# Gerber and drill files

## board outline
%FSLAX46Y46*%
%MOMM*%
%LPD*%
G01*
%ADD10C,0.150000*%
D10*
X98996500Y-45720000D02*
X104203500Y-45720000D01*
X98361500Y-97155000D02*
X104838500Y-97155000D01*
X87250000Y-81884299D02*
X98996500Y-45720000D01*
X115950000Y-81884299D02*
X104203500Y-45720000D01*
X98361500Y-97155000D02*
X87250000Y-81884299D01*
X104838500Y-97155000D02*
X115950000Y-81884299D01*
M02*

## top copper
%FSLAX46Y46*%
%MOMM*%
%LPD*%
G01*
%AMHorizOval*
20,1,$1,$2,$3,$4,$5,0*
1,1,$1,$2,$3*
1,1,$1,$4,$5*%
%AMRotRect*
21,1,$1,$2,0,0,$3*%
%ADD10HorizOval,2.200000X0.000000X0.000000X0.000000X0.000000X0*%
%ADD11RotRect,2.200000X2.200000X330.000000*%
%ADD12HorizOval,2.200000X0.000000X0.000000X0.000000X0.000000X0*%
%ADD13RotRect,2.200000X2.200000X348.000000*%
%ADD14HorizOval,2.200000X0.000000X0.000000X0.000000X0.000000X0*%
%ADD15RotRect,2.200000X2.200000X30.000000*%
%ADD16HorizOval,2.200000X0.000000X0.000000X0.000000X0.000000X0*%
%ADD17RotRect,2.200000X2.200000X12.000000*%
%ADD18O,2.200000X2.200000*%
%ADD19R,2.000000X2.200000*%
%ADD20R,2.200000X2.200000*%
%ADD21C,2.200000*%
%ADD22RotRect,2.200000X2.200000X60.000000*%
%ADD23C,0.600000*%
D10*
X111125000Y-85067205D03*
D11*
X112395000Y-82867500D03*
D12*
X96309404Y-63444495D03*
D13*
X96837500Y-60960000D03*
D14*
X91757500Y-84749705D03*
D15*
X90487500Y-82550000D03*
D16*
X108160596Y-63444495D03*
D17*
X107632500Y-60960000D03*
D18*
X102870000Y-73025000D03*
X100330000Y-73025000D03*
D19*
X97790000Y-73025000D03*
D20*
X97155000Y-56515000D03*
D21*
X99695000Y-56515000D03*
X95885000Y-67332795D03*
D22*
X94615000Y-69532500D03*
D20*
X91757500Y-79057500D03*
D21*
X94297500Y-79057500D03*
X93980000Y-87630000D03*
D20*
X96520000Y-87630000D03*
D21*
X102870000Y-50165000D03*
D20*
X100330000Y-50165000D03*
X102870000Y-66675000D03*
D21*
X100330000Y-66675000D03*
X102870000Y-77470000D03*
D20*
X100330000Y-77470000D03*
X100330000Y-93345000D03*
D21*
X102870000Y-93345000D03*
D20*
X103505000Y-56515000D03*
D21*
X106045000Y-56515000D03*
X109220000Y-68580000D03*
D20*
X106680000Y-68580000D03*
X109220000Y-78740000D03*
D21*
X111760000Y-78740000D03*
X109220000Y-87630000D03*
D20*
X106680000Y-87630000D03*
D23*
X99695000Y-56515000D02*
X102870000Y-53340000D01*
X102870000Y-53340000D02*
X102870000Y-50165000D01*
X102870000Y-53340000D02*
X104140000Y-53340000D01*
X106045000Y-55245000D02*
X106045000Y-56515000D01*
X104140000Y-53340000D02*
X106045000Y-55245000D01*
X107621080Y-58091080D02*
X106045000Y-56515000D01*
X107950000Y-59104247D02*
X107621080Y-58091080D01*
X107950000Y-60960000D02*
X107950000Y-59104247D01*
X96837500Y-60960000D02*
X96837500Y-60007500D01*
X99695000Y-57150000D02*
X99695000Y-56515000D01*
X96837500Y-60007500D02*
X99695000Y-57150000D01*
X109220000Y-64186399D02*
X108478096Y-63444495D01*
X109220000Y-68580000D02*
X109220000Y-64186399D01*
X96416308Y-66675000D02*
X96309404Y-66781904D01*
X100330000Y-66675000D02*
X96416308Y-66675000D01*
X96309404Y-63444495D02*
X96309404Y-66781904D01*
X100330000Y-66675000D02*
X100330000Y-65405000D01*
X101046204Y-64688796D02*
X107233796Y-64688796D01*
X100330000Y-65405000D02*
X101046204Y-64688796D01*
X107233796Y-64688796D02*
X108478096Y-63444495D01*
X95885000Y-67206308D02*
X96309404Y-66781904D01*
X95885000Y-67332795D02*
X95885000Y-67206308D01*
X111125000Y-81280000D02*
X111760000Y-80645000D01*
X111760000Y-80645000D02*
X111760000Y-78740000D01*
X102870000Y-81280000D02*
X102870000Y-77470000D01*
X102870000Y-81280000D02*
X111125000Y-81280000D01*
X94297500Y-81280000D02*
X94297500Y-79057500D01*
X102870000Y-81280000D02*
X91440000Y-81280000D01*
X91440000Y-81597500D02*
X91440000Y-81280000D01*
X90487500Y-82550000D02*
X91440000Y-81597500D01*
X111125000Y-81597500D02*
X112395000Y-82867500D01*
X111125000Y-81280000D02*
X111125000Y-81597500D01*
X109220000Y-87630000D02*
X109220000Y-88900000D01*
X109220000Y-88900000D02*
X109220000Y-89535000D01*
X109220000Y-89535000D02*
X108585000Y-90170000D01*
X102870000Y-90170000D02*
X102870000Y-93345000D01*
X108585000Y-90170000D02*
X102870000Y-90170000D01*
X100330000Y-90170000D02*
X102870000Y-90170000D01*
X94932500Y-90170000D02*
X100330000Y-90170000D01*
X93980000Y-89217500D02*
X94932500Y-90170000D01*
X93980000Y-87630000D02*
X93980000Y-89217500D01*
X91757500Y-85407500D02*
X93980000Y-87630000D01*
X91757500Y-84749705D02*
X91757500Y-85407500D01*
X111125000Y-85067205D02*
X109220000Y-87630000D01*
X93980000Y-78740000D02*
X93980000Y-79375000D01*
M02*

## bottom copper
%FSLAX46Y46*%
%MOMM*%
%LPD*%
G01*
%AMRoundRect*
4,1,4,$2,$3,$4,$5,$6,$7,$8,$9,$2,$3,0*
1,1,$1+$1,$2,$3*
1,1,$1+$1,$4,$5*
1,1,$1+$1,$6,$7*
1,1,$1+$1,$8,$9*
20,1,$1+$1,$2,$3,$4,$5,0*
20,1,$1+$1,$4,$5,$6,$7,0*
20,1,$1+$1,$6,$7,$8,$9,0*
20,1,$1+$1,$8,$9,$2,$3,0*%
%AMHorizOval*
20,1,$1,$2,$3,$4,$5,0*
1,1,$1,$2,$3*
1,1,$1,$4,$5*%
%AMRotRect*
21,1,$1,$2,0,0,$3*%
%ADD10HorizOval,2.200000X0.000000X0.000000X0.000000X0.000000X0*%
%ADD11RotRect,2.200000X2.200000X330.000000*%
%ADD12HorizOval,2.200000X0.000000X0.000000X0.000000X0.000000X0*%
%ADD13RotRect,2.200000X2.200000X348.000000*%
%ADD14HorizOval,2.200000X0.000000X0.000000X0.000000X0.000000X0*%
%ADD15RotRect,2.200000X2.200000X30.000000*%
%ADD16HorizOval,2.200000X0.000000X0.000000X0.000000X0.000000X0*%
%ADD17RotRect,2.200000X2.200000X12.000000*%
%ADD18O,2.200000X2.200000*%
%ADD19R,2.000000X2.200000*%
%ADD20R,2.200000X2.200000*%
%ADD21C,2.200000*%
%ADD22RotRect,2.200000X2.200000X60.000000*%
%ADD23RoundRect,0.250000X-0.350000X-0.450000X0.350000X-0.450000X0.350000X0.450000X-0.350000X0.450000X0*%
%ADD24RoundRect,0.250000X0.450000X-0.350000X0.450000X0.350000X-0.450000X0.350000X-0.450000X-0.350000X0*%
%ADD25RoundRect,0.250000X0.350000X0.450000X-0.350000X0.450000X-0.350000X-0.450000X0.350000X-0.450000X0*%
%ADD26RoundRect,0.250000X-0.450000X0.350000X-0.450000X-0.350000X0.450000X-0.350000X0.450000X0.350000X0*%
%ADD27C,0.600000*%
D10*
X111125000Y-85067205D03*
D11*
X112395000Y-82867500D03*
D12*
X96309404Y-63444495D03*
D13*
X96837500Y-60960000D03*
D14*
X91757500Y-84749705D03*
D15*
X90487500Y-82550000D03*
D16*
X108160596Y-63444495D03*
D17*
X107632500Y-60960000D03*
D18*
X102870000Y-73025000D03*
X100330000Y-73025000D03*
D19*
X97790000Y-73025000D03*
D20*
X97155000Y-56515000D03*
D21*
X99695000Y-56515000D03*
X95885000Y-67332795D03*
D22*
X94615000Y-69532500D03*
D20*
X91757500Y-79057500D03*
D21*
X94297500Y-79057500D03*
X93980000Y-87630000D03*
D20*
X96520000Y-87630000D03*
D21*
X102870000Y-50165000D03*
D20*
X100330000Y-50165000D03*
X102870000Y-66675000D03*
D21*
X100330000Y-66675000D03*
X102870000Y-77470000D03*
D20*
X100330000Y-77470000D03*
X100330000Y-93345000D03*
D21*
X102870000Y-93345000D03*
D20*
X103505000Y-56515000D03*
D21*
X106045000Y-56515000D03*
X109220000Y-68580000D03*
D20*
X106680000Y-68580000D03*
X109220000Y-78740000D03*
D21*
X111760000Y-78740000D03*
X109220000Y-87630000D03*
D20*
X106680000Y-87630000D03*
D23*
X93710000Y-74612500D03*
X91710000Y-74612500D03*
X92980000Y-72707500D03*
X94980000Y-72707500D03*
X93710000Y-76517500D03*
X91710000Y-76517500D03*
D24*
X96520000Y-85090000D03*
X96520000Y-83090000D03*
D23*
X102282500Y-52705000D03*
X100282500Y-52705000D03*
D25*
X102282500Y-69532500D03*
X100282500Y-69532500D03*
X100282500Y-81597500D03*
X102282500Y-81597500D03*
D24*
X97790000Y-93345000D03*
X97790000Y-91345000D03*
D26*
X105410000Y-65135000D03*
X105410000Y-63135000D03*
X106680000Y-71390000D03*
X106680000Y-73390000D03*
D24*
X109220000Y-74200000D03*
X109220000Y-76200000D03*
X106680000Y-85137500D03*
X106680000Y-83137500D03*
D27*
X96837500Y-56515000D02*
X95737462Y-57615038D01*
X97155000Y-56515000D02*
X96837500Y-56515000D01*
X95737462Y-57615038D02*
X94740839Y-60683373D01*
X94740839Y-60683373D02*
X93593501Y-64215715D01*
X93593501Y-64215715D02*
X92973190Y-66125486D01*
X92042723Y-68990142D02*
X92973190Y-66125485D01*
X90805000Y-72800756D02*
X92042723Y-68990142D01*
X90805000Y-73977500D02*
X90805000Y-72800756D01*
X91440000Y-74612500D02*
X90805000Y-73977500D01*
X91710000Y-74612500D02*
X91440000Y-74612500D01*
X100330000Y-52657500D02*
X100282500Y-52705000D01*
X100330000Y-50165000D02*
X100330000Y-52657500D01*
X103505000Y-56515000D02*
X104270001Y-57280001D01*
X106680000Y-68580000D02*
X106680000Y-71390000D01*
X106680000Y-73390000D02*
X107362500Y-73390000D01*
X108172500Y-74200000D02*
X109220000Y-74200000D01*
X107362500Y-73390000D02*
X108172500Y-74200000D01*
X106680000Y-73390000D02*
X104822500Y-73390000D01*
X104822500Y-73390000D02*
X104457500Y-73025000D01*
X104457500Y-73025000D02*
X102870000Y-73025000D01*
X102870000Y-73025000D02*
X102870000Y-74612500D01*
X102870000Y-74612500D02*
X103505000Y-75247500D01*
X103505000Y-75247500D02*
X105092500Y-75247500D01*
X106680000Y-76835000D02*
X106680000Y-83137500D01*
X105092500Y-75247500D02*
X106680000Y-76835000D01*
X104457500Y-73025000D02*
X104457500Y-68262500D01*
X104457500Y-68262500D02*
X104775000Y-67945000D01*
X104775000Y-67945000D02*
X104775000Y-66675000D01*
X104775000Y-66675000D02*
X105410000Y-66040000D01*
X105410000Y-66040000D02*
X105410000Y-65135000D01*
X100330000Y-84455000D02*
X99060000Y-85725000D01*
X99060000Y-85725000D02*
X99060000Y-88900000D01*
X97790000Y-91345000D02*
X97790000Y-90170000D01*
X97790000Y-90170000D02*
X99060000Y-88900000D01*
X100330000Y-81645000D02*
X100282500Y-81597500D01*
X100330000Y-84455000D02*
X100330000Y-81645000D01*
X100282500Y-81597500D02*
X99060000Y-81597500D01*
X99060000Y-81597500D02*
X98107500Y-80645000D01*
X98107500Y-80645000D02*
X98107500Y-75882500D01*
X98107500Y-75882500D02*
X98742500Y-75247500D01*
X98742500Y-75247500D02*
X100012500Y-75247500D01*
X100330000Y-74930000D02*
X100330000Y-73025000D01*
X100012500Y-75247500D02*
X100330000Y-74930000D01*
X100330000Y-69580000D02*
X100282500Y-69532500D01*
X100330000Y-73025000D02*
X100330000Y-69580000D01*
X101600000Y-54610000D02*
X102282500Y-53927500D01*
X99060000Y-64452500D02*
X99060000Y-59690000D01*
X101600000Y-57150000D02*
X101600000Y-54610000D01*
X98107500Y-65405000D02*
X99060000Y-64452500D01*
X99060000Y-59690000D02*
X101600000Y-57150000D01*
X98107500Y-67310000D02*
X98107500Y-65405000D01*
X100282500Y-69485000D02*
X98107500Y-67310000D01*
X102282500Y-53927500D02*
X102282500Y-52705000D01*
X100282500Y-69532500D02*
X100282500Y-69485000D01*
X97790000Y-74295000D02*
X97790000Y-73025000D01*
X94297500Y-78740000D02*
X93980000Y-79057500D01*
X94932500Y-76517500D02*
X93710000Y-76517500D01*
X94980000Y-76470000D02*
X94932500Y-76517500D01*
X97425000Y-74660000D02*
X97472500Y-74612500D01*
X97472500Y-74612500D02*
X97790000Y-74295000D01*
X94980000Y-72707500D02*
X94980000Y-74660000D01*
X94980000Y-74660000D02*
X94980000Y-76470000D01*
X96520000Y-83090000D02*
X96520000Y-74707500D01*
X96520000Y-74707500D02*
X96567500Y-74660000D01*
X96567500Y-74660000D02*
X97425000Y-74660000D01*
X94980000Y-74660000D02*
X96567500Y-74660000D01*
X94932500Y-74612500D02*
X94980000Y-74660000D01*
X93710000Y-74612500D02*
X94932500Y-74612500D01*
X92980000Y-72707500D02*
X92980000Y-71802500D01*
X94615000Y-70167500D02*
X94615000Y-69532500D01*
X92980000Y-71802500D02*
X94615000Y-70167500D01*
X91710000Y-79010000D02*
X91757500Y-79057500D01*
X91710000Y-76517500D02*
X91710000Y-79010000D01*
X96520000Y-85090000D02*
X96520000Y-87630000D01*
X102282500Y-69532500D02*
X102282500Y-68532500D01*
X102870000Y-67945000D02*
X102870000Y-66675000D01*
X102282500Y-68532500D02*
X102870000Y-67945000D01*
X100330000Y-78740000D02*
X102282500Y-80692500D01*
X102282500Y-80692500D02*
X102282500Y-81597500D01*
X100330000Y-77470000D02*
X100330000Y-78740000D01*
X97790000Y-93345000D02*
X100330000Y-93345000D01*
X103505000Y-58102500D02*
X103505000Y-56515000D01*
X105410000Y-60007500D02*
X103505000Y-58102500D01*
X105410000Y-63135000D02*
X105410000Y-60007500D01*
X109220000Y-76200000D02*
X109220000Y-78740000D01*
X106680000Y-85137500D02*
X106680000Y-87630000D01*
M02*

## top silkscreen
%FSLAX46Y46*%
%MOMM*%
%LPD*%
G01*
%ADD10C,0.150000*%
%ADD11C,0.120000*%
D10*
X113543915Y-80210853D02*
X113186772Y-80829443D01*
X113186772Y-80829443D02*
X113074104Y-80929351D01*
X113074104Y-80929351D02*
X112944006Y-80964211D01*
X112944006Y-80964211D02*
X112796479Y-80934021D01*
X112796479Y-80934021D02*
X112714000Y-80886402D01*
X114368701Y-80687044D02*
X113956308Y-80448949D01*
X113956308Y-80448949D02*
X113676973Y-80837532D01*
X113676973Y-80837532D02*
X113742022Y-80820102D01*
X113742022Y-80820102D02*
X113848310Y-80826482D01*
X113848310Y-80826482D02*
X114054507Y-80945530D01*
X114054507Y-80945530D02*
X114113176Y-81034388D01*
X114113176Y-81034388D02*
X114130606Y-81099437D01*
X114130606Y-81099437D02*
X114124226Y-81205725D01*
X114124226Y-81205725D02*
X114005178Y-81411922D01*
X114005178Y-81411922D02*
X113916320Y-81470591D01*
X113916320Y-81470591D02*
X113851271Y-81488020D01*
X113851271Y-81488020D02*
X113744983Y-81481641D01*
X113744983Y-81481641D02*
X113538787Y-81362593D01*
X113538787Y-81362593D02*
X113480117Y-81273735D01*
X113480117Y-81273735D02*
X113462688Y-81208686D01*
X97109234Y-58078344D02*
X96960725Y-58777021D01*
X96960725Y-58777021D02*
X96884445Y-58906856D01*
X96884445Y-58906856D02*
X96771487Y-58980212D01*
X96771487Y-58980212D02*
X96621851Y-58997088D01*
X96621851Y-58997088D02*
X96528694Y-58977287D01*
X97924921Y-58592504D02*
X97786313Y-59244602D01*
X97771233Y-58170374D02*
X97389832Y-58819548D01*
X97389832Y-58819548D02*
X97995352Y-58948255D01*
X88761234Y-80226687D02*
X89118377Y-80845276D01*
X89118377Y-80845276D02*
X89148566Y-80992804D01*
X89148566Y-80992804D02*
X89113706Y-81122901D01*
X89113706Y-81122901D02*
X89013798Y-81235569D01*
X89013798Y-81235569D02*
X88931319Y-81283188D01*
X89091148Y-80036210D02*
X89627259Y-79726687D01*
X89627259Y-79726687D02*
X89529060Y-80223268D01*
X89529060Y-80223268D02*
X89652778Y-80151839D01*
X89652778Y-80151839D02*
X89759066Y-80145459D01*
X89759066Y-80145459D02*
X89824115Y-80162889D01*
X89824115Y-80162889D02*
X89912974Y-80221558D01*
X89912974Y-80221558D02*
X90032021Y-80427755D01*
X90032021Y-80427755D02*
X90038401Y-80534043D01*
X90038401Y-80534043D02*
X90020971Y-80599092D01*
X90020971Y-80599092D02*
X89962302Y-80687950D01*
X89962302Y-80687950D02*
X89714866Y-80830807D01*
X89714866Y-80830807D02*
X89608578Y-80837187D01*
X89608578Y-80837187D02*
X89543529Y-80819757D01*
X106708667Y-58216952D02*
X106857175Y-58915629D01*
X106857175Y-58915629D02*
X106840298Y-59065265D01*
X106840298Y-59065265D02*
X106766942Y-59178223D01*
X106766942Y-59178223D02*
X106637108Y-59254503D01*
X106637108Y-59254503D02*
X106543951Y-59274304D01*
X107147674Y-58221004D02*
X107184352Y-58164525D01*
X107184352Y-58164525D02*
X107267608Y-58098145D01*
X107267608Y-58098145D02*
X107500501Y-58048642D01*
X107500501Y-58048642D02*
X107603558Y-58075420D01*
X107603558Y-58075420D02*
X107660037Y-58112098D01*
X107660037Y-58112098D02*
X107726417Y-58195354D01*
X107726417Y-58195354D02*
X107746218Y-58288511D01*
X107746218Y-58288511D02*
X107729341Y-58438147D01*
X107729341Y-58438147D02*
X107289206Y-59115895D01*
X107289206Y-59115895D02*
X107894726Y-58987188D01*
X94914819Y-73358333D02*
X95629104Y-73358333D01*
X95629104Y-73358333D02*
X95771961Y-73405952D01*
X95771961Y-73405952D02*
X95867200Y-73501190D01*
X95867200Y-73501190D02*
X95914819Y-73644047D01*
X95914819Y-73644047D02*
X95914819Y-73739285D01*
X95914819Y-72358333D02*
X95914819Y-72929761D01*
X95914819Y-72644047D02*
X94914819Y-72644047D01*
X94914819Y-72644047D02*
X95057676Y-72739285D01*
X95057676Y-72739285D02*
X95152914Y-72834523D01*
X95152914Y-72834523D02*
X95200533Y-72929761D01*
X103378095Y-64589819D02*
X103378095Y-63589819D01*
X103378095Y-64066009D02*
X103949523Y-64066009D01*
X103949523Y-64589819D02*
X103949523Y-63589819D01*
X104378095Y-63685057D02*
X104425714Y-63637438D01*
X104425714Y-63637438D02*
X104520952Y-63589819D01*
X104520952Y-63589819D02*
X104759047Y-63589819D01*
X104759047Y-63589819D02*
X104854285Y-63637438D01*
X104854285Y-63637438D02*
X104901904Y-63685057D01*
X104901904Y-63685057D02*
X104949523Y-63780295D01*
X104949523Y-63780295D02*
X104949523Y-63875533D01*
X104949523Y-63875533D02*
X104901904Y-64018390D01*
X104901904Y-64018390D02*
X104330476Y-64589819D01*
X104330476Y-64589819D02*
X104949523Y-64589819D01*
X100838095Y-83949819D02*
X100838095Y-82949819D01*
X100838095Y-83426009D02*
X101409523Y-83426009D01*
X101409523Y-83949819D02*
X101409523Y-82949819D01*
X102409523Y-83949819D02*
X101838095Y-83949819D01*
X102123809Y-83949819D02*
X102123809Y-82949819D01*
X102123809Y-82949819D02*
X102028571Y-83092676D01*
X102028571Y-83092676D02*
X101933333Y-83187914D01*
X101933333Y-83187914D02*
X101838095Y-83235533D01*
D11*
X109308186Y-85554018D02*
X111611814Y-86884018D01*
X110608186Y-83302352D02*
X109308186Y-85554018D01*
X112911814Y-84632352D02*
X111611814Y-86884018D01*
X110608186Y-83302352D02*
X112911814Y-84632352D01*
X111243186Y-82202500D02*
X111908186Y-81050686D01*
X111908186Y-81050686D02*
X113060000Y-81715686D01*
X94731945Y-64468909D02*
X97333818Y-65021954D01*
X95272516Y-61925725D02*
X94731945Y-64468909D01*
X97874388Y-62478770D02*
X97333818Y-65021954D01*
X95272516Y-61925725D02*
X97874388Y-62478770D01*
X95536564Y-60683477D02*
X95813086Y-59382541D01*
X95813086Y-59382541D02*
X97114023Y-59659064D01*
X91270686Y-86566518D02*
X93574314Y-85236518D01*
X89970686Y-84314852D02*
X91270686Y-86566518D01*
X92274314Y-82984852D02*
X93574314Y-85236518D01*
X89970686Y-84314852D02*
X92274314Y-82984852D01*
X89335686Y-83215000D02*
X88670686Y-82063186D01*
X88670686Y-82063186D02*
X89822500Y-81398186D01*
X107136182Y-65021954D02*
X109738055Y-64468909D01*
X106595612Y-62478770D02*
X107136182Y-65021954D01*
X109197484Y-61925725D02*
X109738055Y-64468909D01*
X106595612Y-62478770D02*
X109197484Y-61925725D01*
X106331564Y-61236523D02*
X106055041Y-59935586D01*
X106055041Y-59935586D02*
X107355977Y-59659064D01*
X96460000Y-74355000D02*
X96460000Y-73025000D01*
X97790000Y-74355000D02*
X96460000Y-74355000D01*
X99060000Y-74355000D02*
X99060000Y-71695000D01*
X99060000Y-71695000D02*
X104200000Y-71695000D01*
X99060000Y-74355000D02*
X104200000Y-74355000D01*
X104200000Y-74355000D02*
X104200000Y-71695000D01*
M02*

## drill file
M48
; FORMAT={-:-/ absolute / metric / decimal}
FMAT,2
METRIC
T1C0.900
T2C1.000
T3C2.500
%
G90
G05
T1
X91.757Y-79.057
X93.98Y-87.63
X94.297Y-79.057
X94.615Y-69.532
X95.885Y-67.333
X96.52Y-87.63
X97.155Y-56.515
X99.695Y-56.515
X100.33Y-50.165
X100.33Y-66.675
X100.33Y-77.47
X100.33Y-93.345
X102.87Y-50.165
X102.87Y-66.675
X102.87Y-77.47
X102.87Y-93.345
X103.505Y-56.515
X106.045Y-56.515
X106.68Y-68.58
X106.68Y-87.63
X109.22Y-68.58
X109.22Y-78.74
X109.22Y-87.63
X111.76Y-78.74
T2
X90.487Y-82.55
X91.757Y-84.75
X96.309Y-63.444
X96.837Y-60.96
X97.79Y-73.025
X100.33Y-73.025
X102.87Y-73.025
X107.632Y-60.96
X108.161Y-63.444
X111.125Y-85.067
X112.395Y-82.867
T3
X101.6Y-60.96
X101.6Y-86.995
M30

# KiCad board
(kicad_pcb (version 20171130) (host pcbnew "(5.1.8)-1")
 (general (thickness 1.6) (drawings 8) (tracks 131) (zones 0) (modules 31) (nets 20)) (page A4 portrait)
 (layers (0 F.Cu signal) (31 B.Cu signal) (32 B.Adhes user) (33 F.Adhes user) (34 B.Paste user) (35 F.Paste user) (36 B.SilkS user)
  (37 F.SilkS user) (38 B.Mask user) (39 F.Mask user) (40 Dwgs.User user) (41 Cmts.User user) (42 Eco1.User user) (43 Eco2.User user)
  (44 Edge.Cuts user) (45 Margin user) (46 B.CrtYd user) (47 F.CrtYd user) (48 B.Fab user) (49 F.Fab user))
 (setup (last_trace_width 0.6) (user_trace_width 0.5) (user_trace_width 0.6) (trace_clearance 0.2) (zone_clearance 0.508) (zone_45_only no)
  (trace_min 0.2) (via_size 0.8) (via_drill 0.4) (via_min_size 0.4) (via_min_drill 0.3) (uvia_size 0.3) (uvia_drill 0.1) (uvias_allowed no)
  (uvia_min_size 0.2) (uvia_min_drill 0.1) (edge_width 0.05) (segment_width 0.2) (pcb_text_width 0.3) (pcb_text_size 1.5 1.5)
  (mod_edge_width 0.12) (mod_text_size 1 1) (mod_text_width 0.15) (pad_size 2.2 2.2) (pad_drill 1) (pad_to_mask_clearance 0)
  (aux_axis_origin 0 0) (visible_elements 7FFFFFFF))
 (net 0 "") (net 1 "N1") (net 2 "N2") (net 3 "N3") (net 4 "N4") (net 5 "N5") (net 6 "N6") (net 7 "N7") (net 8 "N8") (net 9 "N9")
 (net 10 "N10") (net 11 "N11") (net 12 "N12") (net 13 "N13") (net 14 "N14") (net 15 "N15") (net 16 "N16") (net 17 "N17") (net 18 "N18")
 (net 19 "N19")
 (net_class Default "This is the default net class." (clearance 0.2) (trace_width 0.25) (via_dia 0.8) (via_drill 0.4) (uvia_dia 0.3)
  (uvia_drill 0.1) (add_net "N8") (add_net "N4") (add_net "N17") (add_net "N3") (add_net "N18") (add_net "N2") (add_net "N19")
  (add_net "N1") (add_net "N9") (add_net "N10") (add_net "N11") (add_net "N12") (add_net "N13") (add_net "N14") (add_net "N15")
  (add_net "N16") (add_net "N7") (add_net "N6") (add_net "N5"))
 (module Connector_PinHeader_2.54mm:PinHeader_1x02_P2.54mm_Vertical (layer F.Cu) (at 112.395 82.8675 330)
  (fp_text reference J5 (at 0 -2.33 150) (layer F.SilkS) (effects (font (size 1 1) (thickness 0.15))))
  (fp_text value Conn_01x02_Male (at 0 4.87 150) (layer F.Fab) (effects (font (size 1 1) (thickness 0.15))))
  (fp_line (start -1.33 3.87) (end 1.33 3.87) (layer F.SilkS) (width 0.12))
  (fp_line (start -1.33 1.27) (end -1.33 3.87) (layer F.SilkS) (width 0.12))
  (fp_line (start 1.33 1.27) (end 1.33 3.87) (layer F.SilkS) (width 0.12))
  (fp_line (start -1.33 1.27) (end 1.33 1.27) (layer F.SilkS) (width 0.12))
  (fp_line (start -1.33 0) (end -1.33 -1.33) (layer F.SilkS) (width 0.12))
  (fp_line (start -1.33 -1.33) (end 0 -1.33) (layer F.SilkS) (width 0.12))
  (pad 2 thru_hole oval (at 0 2.54 330) (size 2.2 2.2) (drill 1) (layers *.Cu *.Mask) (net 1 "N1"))
  (pad 1 thru_hole rect (at 0 0 330) (size 2.2 2.2) (drill 1) (layers *.Cu *.Mask) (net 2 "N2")))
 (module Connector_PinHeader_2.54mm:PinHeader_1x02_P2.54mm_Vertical (layer F.Cu) (at 96.8375 60.96 348)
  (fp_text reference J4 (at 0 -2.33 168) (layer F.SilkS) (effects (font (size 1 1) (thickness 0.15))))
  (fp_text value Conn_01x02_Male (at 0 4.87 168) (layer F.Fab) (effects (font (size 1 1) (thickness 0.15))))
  (fp_line (start -1.33 3.87) (end 1.33 3.87) (layer F.SilkS) (width 0.12))
  (fp_line (start -1.33 1.27) (end -1.33 3.87) (layer F.SilkS) (width 0.12))
  (fp_line (start 1.33 1.27) (end 1.33 3.87) (layer F.SilkS) (width 0.12))
  (fp_line (start -1.33 1.27) (end 1.33 1.27) (layer F.SilkS) (width 0.12))
  (fp_line (start -1.33 0) (end -1.33 -1.33) (layer F.SilkS) (width 0.12))
  (fp_line (start -1.33 -1.33) (end 0 -1.33) (layer F.SilkS) (width 0.12))
  (pad 2 thru_hole oval (at 0 2.54 348) (size 2.2 2.2) (drill 1) (layers *.Cu *.Mask) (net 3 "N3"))
  (pad 1 thru_hole rect (at 0 0 348) (size 2.2 2.2) (drill 1) (layers *.Cu *.Mask) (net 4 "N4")))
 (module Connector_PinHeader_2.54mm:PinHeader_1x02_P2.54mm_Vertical (layer F.Cu) (at 90.4875 82.55 30)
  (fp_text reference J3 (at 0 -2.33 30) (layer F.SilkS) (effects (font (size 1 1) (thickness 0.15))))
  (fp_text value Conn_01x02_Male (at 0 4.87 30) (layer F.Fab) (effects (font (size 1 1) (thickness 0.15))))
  (fp_line (start -1.33 3.87) (end 1.33 3.87) (layer F.SilkS) (width 0.12))
  (fp_line (start -1.33 1.27) (end -1.33 3.87) (layer F.SilkS) (width 0.12))
  (fp_line (start 1.33 1.27) (end 1.33 3.87) (layer F.SilkS) (width 0.12))
  (fp_line (start -1.33 1.27) (end 1.33 1.27) (layer F.SilkS) (width 0.12))
  (fp_line (start -1.33 0) (end -1.33 -1.33) (layer F.SilkS) (width 0.12))
  (fp_line (start -1.33 -1.33) (end 0 -1.33) (layer F.SilkS) (width 0.12))
  (pad 2 thru_hole oval (at 0 2.54 30) (size 2.2 2.2) (drill 1) (layers *.Cu *.Mask) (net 1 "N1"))
  (pad 1 thru_hole rect (at 0 0 30) (size 2.2 2.2) (drill 1) (layers *.Cu *.Mask) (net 2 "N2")))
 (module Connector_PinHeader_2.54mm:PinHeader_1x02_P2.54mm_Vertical (layer F.Cu) (at 107.6325 60.96 12)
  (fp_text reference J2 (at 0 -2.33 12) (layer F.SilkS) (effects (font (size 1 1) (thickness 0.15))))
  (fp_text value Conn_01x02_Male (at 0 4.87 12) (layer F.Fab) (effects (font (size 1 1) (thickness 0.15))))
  (fp_line (start -1.33 3.87) (end 1.33 3.87) (layer F.SilkS) (width 0.12))
  (fp_line (start -1.33 1.27) (end -1.33 3.87) (layer F.SilkS) (width 0.12))
  (fp_line (start 1.33 1.27) (end 1.33 3.87) (layer F.SilkS) (width 0.12))
  (fp_line (start -1.33 1.27) (end 1.33 1.27) (layer F.SilkS) (width 0.12))
  (fp_line (start -1.33 0) (end -1.33 -1.33) (layer F.SilkS) (width 0.12))
  (fp_line (start -1.33 -1.33) (end 0 -1.33) (layer F.SilkS) (width 0.12))
  (pad 2 thru_hole oval (at 0 2.54 12) (size 2.2 2.2) (drill 1) (layers *.Cu *.Mask) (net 3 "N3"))
  (pad 1 thru_hole rect (at 0 0 12) (size 2.2 2.2) (drill 1) (layers *.Cu *.Mask) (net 4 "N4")))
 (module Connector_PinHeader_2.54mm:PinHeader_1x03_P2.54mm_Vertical (layer F.Cu) (at 97.79 73.025 90)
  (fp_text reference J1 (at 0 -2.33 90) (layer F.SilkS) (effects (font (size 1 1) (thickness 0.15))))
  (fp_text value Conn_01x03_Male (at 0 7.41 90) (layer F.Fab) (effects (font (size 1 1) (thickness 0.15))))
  (fp_line (start -1.33 -1.33) (end 0 -1.33) (layer F.SilkS) (width 0.12))
  (fp_line (start -1.33 0) (end -1.33 -1.33) (layer F.SilkS) (width 0.12))
  (fp_line (start -1.33 1.27) (end 1.33 1.27) (layer F.SilkS) (width 0.12))
  (fp_line (start 1.33 1.27) (end 1.33 6.41) (layer F.SilkS) (width 0.12))
  (fp_line (start -1.33 1.27) (end -1.33 6.41) (layer F.SilkS) (width 0.12))
  (fp_line (start -1.33 6.41) (end 1.33 6.41) (layer F.SilkS) (width 0.12))
  (pad 3 thru_hole oval (at 0 5.08 90) (size 2.2 2.2) (drill 1) (layers *.Cu *.Mask) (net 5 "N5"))
  (pad 2 thru_hole oval (at 0 2.54 90) (size 2.2 2.2) (drill 1) (layers *.Cu *.Mask) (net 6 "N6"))
  (pad 1 thru_hole rect (at 0 0 90) (size 2.2 2) (drill 1) (layers *.Cu *.Mask) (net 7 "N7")))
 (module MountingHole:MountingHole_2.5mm (layer F.Cu) (at 101.6 60.96)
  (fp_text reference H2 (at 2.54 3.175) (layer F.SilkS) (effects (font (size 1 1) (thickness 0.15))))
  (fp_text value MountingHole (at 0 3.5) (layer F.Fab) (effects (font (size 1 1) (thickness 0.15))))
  (pad 1 np_thru_hole circle (at 0 0) (size 2.5 2.5) (drill 2.5) (layers *.Cu *.Mask)))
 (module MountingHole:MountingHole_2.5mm (layer F.Cu) (at 101.6 86.995)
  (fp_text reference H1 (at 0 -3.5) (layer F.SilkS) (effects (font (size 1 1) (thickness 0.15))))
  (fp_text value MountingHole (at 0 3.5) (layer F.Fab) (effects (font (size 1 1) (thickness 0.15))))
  (pad 1 np_thru_hole circle (at 0 0) (size 2.5 2.5) (drill 2.5) (layers *.Cu *.Mask)))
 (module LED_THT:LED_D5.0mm (layer B.Cu) (at 97.155 56.515)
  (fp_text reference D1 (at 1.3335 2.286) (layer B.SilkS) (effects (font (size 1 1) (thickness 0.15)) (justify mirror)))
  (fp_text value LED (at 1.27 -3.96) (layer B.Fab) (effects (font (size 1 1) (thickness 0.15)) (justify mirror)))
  (pad 1 thru_hole rect (at 0 0) (size 2.2 2.2) (drill 0.9) (layers *.Cu *.Mask) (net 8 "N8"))
  (pad 2 thru_hole circle (at 2.54 0) (size 2.2 2.2) (drill 0.9) (layers *.Cu *.Mask) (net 4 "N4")))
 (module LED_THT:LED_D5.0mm (layer B.Cu) (at 94.615 69.5325 60)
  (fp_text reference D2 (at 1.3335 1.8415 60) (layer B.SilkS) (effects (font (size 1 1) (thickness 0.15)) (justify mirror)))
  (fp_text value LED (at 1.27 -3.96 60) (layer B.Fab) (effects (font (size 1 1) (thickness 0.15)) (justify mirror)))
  (pad 2 thru_hole circle (at 2.54 0 60) (size 2.2 2.2) (drill 0.9) (layers *.Cu *.Mask) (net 3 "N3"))
  (pad 1 thru_hole rect (at 0 0 60) (size 2.2 2.2) (drill 0.9) (layers *.Cu *.Mask) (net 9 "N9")))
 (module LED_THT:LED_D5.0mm (layer B.Cu) (at 91.7575 79.0575)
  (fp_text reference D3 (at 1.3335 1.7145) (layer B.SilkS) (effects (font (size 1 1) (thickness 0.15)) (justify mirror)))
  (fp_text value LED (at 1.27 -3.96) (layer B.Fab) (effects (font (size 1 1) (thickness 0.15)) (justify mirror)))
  (pad 1 thru_hole rect (at 0 0) (size 2.2 2.2) (drill 0.9) (layers *.Cu *.Mask) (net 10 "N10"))
  (pad 2 thru_hole circle (at 2.54 0) (size 2.2 2.2) (drill 0.9) (layers *.Cu *.Mask) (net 2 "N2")))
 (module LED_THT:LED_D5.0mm (layer B.Cu) (at 96.52 87.63 180)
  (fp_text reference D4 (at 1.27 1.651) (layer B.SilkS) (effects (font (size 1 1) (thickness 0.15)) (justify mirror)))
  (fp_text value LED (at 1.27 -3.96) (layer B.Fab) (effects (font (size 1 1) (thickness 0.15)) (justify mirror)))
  (pad 2 thru_hole circle (at 2.54 0 180) (size 2.2 2.2) (drill 0.9) (layers *.Cu *.Mask) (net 1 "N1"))
  (pad 1 thru_hole rect (at 0 0 180) (size 2.2 2.2) (drill 0.9) (layers *.Cu *.Mask) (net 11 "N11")))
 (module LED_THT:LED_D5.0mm (layer B.Cu) (at 100.33 50.165)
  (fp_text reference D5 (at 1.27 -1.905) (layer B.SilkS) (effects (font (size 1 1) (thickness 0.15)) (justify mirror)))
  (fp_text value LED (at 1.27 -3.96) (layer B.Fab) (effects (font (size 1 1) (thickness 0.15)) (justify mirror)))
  (pad 2 thru_hole circle (at 2.54 0) (size 2.2 2.2) (drill 0.9) (layers *.Cu *.Mask) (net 4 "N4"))
  (pad 1 thru_hole rect (at 0 0) (size 2.2 2.2) (drill 0.9) (layers *.Cu *.Mask) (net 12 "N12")))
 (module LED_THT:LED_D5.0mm (layer B.Cu) (at 102.87 66.675 180)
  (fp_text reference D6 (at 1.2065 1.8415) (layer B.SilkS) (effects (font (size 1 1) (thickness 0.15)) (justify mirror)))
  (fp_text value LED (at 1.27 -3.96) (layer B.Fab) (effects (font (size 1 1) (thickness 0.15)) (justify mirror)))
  (pad 1 thru_hole rect (at 0 0 180) (size 2.2 2.2) (drill 0.9) (layers *.Cu *.Mask) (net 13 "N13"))
  (pad 2 thru_hole circle (at 2.54 0 180) (size 2.2 2.2) (drill 0.9) (layers *.Cu *.Mask) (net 3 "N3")))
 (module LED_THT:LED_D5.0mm (layer B.Cu) (at 100.33 77.47)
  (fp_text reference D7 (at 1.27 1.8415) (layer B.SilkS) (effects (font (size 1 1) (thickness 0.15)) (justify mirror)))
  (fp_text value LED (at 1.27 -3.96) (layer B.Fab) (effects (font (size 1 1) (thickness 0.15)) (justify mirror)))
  (pad 2 thru_hole circle (at 2.54 0) (size 2.2 2.2) (drill 0.9) (layers *.Cu *.Mask) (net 2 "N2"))
  (pad 1 thru_hole rect (at 0 0) (size 2.2 2.2) (drill 0.9) (layers *.Cu *.Mask) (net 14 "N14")))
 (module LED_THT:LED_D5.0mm (layer B.Cu) (at 100.33 93.345)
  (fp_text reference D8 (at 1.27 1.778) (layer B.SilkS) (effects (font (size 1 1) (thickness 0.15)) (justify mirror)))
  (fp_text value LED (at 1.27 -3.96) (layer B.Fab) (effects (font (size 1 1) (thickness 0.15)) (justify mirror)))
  (pad 1 thru_hole rect (at 0 0) (size 2.2 2.2) (drill 0.9) (layers *.Cu *.Mask) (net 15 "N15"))
  (pad 2 thru_hole circle (at 2.54 0) (size 2.2 2.2) (drill 0.9) (layers *.Cu *.Mask) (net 1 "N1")))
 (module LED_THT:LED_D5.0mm (layer B.Cu) (at 103.505 56.515)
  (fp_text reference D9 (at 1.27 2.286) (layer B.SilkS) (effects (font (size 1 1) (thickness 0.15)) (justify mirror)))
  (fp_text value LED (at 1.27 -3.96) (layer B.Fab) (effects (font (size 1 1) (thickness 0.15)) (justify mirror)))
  (pad 1 thru_hole rect (at 0 0) (size 2.2 2.2) (drill 0.9) (layers *.Cu *.Mask) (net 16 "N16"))
  (pad 2 thru_hole circle (at 2.54 0) (size 2.2 2.2) (drill 0.9) (layers *.Cu *.Mask) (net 4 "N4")))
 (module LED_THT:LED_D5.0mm (layer B.Cu) (at 106.68 68.58)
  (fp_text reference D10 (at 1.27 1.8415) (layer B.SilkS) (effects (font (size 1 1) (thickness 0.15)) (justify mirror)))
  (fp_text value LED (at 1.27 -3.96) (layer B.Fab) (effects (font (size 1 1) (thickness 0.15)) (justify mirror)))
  (pad 2 thru_hole circle (at 2.54 0) (size 2.2 2.2) (drill 0.9) (layers *.Cu *.Mask) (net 3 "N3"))
  (pad 1 thru_hole rect (at 0 0) (size 2.2 2.2) (drill 0.9) (layers *.Cu *.Mask) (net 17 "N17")))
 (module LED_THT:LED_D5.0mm (layer B.Cu) (at 109.22 78.74)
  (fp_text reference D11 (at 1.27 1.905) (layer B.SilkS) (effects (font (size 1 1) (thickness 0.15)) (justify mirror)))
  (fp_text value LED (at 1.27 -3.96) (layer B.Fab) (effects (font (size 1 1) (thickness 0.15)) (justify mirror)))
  (pad 1 thru_hole rect (at 0 0) (size 2.2 2.2) (drill 0.9) (layers *.Cu *.Mask) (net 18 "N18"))
  (pad 2 thru_hole circle (at 2.54 0) (size 2.2 2.2) (drill 0.9) (layers *.Cu *.Mask) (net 2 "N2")))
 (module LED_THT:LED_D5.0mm (layer B.Cu) (at 106.68 87.63)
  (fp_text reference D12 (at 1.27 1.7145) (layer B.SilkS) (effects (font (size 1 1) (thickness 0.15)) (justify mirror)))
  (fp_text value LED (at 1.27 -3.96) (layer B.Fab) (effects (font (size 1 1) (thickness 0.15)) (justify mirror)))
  (pad 2 thru_hole circle (at 2.54 0) (size 2.2 2.2) (drill 0.9) (layers *.Cu *.Mask) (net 1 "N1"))
  (pad 1 thru_hole rect (at 0 0) (size 2.2 2.2) (drill 0.9) (layers *.Cu *.Mask) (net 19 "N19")))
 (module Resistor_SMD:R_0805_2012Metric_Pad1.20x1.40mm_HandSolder (layer B.Cu) (at 92.71 74.6125)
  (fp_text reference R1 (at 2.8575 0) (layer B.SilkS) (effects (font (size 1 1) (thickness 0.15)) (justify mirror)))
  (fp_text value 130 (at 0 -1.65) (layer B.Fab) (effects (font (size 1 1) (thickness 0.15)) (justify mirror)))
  (pad 2 smd roundrect (at 1 0) (size 1.2 1.4) (layers B.Cu B.Paste B.Mask) (roundrect_rratio 0.208333) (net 7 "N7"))
  (pad 1 smd roundrect (at -1 0) (size 1.2 1.4) (layers B.Cu B.Paste B.Mask) (roundrect_rratio 0.208333) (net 8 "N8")))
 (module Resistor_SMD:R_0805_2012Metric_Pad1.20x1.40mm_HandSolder (layer B.Cu) (at 93.98 72.7075)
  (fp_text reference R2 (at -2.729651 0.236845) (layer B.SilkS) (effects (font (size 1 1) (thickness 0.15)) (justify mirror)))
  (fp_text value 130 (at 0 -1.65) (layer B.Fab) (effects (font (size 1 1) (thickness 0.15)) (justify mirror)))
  (pad 1 smd roundrect (at -1 0) (size 1.2 1.4) (layers B.Cu B.Paste B.Mask) (roundrect_rratio 0.208333) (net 9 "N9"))
  (pad 2 smd roundrect (at 1 0) (size 1.2 1.4) (layers B.Cu B.Paste B.Mask) (roundrect_rratio 0.208333) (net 7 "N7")))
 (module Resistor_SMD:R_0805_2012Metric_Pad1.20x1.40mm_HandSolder (layer B.Cu) (at 92.71 76.5175)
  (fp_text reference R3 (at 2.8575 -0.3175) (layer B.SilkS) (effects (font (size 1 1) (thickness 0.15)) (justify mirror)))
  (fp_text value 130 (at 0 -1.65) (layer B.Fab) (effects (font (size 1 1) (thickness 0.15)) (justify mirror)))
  (pad 2 smd roundrect (at 1 0) (size 1.2 1.4) (layers B.Cu B.Paste B.Mask) (roundrect_rratio 0.208333) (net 7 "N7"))
  (pad 1 smd roundrect (at -1 0) (size 1.2 1.4) (layers B.Cu B.Paste B.Mask) (roundrect_rratio 0.208333) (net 10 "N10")))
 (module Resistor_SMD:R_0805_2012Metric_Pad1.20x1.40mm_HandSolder (layer B.Cu) (at 96.52 84.09 90)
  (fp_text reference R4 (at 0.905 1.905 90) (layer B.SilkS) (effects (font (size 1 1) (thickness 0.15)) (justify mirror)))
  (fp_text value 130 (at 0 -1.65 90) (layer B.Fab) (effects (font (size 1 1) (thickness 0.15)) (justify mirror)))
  (pad 1 smd roundrect (at -1 0 90) (size 1.2 1.4) (layers B.Cu B.Paste B.Mask) (roundrect_rratio 0.208333) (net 11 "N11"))
  (pad 2 smd roundrect (at 1 0 90) (size 1.2 1.4) (layers B.Cu B.Paste B.Mask) (roundrect_rratio 0.208333) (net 7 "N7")))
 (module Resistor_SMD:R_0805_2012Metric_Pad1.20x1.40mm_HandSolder (layer B.Cu) (at 101.2825 52.705)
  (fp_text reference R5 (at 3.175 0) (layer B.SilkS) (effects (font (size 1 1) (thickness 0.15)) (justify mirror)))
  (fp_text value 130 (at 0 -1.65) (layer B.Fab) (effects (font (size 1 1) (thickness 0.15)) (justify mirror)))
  (pad 2 smd roundrect (at 1 0) (size 1.2 1.4) (layers B.Cu B.Paste B.Mask) (roundrect_rratio 0.208333) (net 6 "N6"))
  (pad 1 smd roundrect (at -1 0) (size 1.2 1.4) (layers B.Cu B.Paste B.Mask) (roundrect_rratio 0.208333) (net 12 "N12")))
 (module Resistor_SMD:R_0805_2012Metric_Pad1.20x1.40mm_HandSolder (layer B.Cu) (at 101.2825 69.5325 180)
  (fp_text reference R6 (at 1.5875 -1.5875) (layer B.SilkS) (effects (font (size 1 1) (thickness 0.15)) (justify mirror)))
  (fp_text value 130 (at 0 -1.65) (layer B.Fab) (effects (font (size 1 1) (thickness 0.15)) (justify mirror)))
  (pad 1 smd roundrect (at -1 0 180) (size 1.2 1.4) (layers B.Cu B.Paste B.Mask) (roundrect_rratio 0.208333) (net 13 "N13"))
  (pad 2 smd roundrect (at 1 0 180) (size 1.2 1.4) (layers B.Cu B.Paste B.Mask) (roundrect_rratio 0.208333) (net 6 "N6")))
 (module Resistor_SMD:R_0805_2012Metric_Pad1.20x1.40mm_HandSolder (layer B.Cu) (at 101.2825 81.5975 180)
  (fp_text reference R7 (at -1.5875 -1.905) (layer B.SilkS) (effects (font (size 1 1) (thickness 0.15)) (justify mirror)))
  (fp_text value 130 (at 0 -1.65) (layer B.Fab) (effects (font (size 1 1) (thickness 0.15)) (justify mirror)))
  (pad 2 smd roundrect (at 1 0 180) (size 1.2 1.4) (layers B.Cu B.Paste B.Mask) (roundrect_rratio 0.208333) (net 6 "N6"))
  (pad 1 smd roundrect (at -1 0 180) (size 1.2 1.4) (layers B.Cu B.Paste B.Mask) (roundrect_rratio 0.208333) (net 14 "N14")))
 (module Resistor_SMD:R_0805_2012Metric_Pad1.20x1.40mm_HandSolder (layer B.Cu) (at 97.79 92.345 90)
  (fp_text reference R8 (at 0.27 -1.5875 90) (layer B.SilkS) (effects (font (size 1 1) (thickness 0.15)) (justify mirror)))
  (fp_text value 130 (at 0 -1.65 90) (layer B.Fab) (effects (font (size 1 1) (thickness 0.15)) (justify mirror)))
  (pad 1 smd roundrect (at -1 0 90) (size 1.2 1.4) (layers B.Cu B.Paste B.Mask) (roundrect_rratio 0.208333) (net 15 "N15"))
  (pad 2 smd roundrect (at 1 0 90) (size 1.2 1.4) (layers B.Cu B.Paste B.Mask) (roundrect_rratio 0.208333) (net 6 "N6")))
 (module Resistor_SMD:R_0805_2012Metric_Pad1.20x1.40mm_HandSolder (layer B.Cu) (at 105.41 64.135 270)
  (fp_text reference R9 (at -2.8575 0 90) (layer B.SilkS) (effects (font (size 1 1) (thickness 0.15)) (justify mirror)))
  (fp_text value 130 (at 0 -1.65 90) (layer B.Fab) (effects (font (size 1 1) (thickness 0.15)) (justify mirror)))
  (pad 2 smd roundrect (at 1 0 270) (size 1.2 1.4) (layers B.Cu B.Paste B.Mask) (roundrect_rratio 0.208333) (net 5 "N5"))
  (pad 1 smd roundrect (at -1 0 270) (size 1.2 1.4) (layers B.Cu B.Paste B.Mask) (roundrect_rratio 0.208333) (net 16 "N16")))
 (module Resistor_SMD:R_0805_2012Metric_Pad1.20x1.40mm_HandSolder (layer B.Cu) (at 106.68 72.39 270)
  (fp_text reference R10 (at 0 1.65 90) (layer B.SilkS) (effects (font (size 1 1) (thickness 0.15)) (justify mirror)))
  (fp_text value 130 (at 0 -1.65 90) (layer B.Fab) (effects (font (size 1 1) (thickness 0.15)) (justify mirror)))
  (pad 1 smd roundrect (at -1 0 270) (size 1.2 1.4) (layers B.Cu B.Paste B.Mask) (roundrect_rratio 0.208333) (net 17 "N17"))
  (pad 2 smd roundrect (at 1 0 270) (size 1.2 1.4) (layers B.Cu B.Paste B.Mask) (roundrect_rratio 0.208333) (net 5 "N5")))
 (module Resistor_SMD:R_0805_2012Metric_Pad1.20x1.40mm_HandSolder (layer B.Cu) (at 109.22 75.2 90)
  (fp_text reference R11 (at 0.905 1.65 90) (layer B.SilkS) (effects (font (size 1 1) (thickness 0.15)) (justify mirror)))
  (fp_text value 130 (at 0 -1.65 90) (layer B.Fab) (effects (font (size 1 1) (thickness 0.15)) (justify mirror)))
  (pad 2 smd roundrect (at 1 0 90) (size 1.2 1.4) (layers B.Cu B.Paste B.Mask) (roundrect_rratio 0.208333) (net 5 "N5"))
  (pad 1 smd roundrect (at -1 0 90) (size 1.2 1.4) (layers B.Cu B.Paste B.Mask) (roundrect_rratio 0.208333) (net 18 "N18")))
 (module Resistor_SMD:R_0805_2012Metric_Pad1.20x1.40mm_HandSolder (layer B.Cu) (at 106.68 84.1375 90)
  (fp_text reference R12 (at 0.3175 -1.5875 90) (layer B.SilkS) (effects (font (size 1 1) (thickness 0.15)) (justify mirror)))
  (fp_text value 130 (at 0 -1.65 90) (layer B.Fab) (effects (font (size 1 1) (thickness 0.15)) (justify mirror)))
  (pad 1 smd roundrect (at -1 0 90) (size 1.2 1.4) (layers B.Cu B.Paste B.Mask) (roundrect_rratio 0.208333) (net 19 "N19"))
  (pad 2 smd roundrect (at 1 0 90) (size 1.2 1.4) (layers B.Cu B.Paste B.Mask) (roundrect_rratio 0.208333) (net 5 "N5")))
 (gr_line (start 98.9965 45.72) (end 104.2035 45.72) (layer Edge.Cuts) (width 0.15))
 (gr_line (start 98.3615 97.155) (end 104.8385 97.155) (layer Edge.Cuts) (width 0.15))
 (gr_line (start 87.25 81.884299) (end 98.9965 45.72) (layer Edge.Cuts) (width 0.15))
 (gr_line (start 115.95 81.884299) (end 104.2035 45.72) (layer Edge.Cuts) (width 0.15))
 (gr_line (start 98.3615 97.155) (end 87.25 81.884299) (layer Edge.Cuts) (width 0.15))
 (gr_line (start 104.8385 97.155) (end 115.95 81.884299) (layer Edge.Cuts) (width 0.15))
 (segment (start 96.8375 56.515) (end 95.737462 57.615038) (width 0.6) (layer B.Cu) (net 8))
 (segment (start 97.155 56.515) (end 96.8375 56.515) (width 0.6) (layer B.Cu) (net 8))
 (segment (start 95.737462 57.615038) (end 94.740839 60.683373) (width 0.6) (layer B.Cu) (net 8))
 (segment (start 94.740839 60.683373) (end 93.593501 64.215715) (width 0.6) (layer B.Cu) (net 8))
 (segment (start 93.593501 64.215715) (end 92.97319 66.125486) (width 0.6) (layer B.Cu) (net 8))
 (segment (start 92.042723 68.990142) (end 92.97319 66.125485) (width 0.6) (layer B.Cu) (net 8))
 (segment (start 90.805 72.800756) (end 92.042723 68.990142) (width 0.6) (layer B.Cu) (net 8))
 (segment (start 90.805 73.9775) (end 90.805 72.800756) (width 0.6) (layer B.Cu) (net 8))
 (segment (start 91.44 74.6125) (end 90.805 73.9775) (width 0.6) (layer B.Cu) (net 8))
 (segment (start 91.71 74.6125) (end 91.44 74.6125) (width 0.6) (layer B.Cu) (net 8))
 (segment (start 99.695 56.515) (end 102.87 53.34) (width 0.6) (layer F.Cu) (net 4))
 (segment (start 102.87 53.34) (end 102.87 50.165) (width 0.6) (layer F.Cu) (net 4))
 (segment (start 102.87 53.34) (end 104.14 53.34) (width 0.6) (layer F.Cu) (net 4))
 (segment (start 106.045 55.245) (end 106.045 56.515) (width 0.6) (layer F.Cu) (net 4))
 (segment (start 104.14 53.34) (end 106.045 55.245) (width 0.6) (layer F.Cu) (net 4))
 (segment (start 107.62108 58.09108) (end 106.045 56.515) (width 0.6) (layer F.Cu) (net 4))
 (segment (start 107.95 59.104247) (end 107.62108 58.09108) (width 0.6) (layer F.Cu) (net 4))
 (segment (start 107.95 60.96) (end 107.95 59.104247) (width 0.6) (layer F.Cu) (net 4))
 (segment (start 96.8375 60.96) (end 96.8375 60.0075) (width 0.6) (layer F.Cu) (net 4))
 (segment (start 99.695 57.15) (end 99.695 56.515) (width 0.6) (layer F.Cu) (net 4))
 (segment (start 96.8375 60.0075) (end 99.695 57.15) (width 0.6) (layer F.Cu) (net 4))
 (segment (start 100.33 52.6575) (end 100.2825 52.705) (width 0.6) (layer B.Cu) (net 12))
 (segment (start 100.33 50.165) (end 100.33 52.6575) (width 0.6) (layer B.Cu) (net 12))
 (segment (start 109.22 64.186399) (end 108.478096 63.444495) (width 0.6) (layer F.Cu) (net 3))
 (segment (start 109.22 68.58) (end 109.22 64.186399) (width 0.6) (layer F.Cu) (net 3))
 (segment (start 96.416308 66.675) (end 96.309404 66.781904) (width 0.6) (layer F.Cu) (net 3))
 (segment (start 100.33 66.675) (end 96.416308 66.675) (width 0.6) (layer F.Cu) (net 3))
 (segment (start 96.309404 63.444495) (end 96.309404 66.781904) (width 0.6) (layer F.Cu) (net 3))
 (segment (start 100.33 66.675) (end 100.33 65.405) (width 0.6) (layer F.Cu) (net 3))
 (segment (start 101.046204 64.688796) (end 107.233796 64.688796) (width 0.6) (layer F.Cu) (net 3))
 (segment (start 100.33 65.405) (end 101.046204 64.688796) (width 0.6) (layer F.Cu) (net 3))
 (segment (start 107.233796 64.688796) (end 108.478096 63.444495) (width 0.6) (layer F.Cu) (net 3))
 (segment (start 95.885 67.206308) (end 96.309404 66.781904) (width 0.6) (layer F.Cu) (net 3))
 (segment (start 95.885 67.332795) (end 95.885 67.206308) (width 0.6) (layer F.Cu) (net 3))
 (segment (start 103.505 56.515) (end 104.270001 57.280001) (width 0.6) (layer B.Cu) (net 16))
 (segment (start 106.68 68.58) (end 106.68 71.39) (width 0.6) (layer B.Cu) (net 17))
 (segment (start 111.125 81.28) (end 111.76 80.645) (width 0.6) (layer F.Cu) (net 2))
 (segment (start 111.76 80.645) (end 111.76 78.74) (width 0.6) (layer F.Cu) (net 2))
 (segment (start 102.87 81.28) (end 102.87 77.47) (width 0.6) (layer F.Cu) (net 2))
 (segment (start 102.87 81.28) (end 111.125 81.28) (width 0.6) (layer F.Cu) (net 2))
 (segment (start 94.2975 81.28) (end 94.2975 79.0575) (width 0.6) (layer F.Cu) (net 2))
 (segment (start 102.87 81.28) (end 91.44 81.28) (width 0.6) (layer F.Cu) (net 2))
 (segment (start 91.44 81.5975) (end 91.44 81.28) (width 0.6) (layer F.Cu) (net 2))
 (segment (start 90.4875 82.55) (end 91.44 81.5975) (width 0.6) (layer F.Cu) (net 2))
 (segment (start 111.125 81.5975) (end 112.395 82.8675) (width 0.6) (layer F.Cu) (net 2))
 (segment (start 111.125 81.28) (end 111.125 81.5975) (width 0.6) (layer F.Cu) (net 2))
 (segment (start 109.22 87.63) (end 109.22 88.9) (width 0.6) (layer F.Cu) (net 1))
 (segment (start 109.22 88.9) (end 109.22 89.535) (width 0.6) (layer F.Cu) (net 1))
 (segment (start 109.22 89.535) (end 108.585 90.17) (width 0.6) (layer F.Cu) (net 1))
 (segment (start 102.87 90.17) (end 102.87 93.345) (width 0.6) (layer F.Cu) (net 1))
 (segment (start 108.585 90.17) (end 102.87 90.17) (width 0.6) (layer F.Cu) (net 1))
 (segment (start 100.33 90.17) (end 102.87 90.17) (width 0.6) (layer F.Cu) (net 1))
 (segment (start 94.9325 90.17) (end 100.33 90.17) (width 0.6) (layer F.Cu) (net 1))
 (segment (start 93.98 89.2175) (end 94.9325 90.17) (width 0.6) (layer F.Cu) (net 1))
 (segment (start 93.98 87.63) (end 93.98 89.2175) (width 0.6) (layer F.Cu) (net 1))
 (segment (start 91.7575 85.4075) (end 93.98 87.63) (width 0.6) (layer F.Cu) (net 1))
 (segment (start 91.7575 84.749705) (end 91.7575 85.4075) (width 0.6) (layer F.Cu) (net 1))
 (segment (start 111.125 85.067205) (end 109.22 87.63) (width 0.6) (layer F.Cu) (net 1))
 (segment (start 106.68 73.39) (end 107.3625 73.39) (width 0.6) (layer B.Cu) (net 5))
 (segment (start 108.1725 74.2) (end 109.22 74.2) (width 0.6) (layer B.Cu) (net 5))
 (segment (start 107.3625 73.39) (end 108.1725 74.2) (width 0.6) (layer B.Cu) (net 5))
 (segment (start 106.68 73.39) (end 104.8225 73.39) (width 0.6) (layer B.Cu) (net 5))
 (segment (start 104.8225 73.39) (end 104.4575 73.025) (width 0.6) (layer B.Cu) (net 5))
 (segment (start 104.4575 73.025) (end 102.87 73.025) (width 0.6) (layer B.Cu) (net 5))
 (segment (start 102.87 73.025) (end 102.87 74.6125) (width 0.6) (layer B.Cu) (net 5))
 (segment (start 102.87 74.6125) (end 103.505 75.2475) (width 0.6) (layer B.Cu) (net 5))
 (segment (start 103.505 75.2475) (end 105.0925 75.2475) (width 0.6) (layer B.Cu) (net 5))
 (segment (start 106.68 76.835) (end 106.68 83.1375) (width 0.6) (layer B.Cu) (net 5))
 (segment (start 105.0925 75.2475) (end 106.68 76.835) (width 0.6) (layer B.Cu) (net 5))
 (segment (start 104.4575 73.025) (end 104.4575 68.2625) (width 0.6) (layer B.Cu) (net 5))
 (segment (start 104.4575 68.2625) (end 104.775 67.945) (width 0.6) (layer B.Cu) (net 5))
 (segment (start 104.775 67.945) (end 104.775 66.675) (width 0.6) (layer B.Cu) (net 5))
 (segment (start 104.775 66.675) (end 105.41 66.04) (width 0.6) (layer B.Cu) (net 5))
 (segment (start 105.41 66.04) (end 105.41 65.135) (width 0.6) (layer B.Cu) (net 5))
 (segment (start 100.33 84.455) (end 99.06 85.725) (width 0.6) (layer B.Cu) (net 6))
 (segment (start 99.06 85.725) (end 99.06 88.9) (width 0.6) (layer B.Cu) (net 6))
 (segment (start 97.79 91.345) (end 97.79 90.17) (width 0.6) (layer B.Cu) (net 6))
 (segment (start 97.79 90.17) (end 99.06 88.9) (width 0.6) (layer B.Cu) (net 6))
 (segment (start 100.33 81.645) (end 100.2825 81.5975) (width 0.6) (layer B.Cu) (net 6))
 (segment (start 100.33 84.455) (end 100.33 81.645) (width 0.6) (layer B.Cu) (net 6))
 (segment (start 100.2825 81.5975) (end 99.06 81.5975) (width 0.6) (layer B.Cu) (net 6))
 (segment (start 99.06 81.5975) (end 98.1075 80.645) (width 0.6) (layer B.Cu) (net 6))
 (segment (start 98.1075 80.645) (end 98.1075 75.8825) (width 0.6) (layer B.Cu) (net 6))
 (segment (start 98.1075 75.8825) (end 98.7425 75.2475) (width 0.6) (layer B.Cu) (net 6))
 (segment (start 98.7425 75.2475) (end 100.0125 75.2475) (width 0.6) (layer B.Cu) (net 6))
 (segment (start 100.33 74.93) (end 100.33 73.025) (width 0.6) (layer B.Cu) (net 6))
 (segment (start 100.0125 75.2475) (end 100.33 74.93) (width 0.6) (layer B.Cu) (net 6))
 (segment (start 100.33 69.58) (end 100.2825 69.5325) (width 0.6) (layer B.Cu) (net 6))
 (segment (start 100.33 73.025) (end 100.33 69.58) (width 0.6) (layer B.Cu) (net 6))
 (segment (start 101.6 54.61) (end 102.2825 53.9275) (width 0.6) (layer B.Cu) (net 6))
 (segment (start 99.06 64.4525) (end 99.06 59.69) (width 0.6) (layer B.Cu) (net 6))
 (segment (start 101.6 57.15) (end 101.6 54.61) (width 0.6) (layer B.Cu) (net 6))
 (segment (start 98.1075 65.405) (end 99.06 64.4525) (width 0.6) (layer B.Cu) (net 6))
 (segment (start 99.06 59.69) (end 101.6 57.15) (width 0.6) (layer B.Cu) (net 6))
 (segment (start 98.1075 67.31) (end 98.1075 65.405) (width 0.6) (layer B.Cu) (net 6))
 (segment (start 100.2825 69.485) (end 98.1075 67.31) (width 0.6) (layer B.Cu) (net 6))
 (segment (start 102.2825 53.9275) (end 102.2825 52.705) (width 0.6) (layer B.Cu) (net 6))
 (segment (start 100.2825 69.5325) (end 100.2825 69.485) (width 0.6) (layer B.Cu) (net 6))
 (segment (start 97.79 74.295) (end 97.79 73.025) (width 0.6) (layer B.Cu) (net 7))
 (segment (start 93.98 78.74) (end 93.98 79.375) (width 0.6) (layer F.Cu) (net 2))
 (segment (start 94.2975 78.74) (end 93.98 79.0575) (width 0.6) (layer B.Cu) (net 2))
 (segment (start 94.9325 76.5175) (end 93.71 76.5175) (width 0.6) (layer B.Cu) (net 7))
 (segment (start 94.98 76.47) (end 94.9325 76.5175) (width 0.6) (layer B.Cu) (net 7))
 (segment (start 97.425 74.66) (end 97.4725 74.6125) (width 0.6) (layer B.Cu) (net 7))
 (segment (start 97.4725 74.6125) (end 97.79 74.295) (width 0.6) (layer B.Cu) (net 7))
 (segment (start 94.98 72.7075) (end 94.98 74.66) (width 0.6) (layer B.Cu) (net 7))
 (segment (start 94.98 74.66) (end 94.98 76.47) (width 0.6) (layer B.Cu) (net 7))
 (segment (start 96.52 83.09) (end 96.52 74.7075) (width 0.6) (layer B.Cu) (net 7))
 (segment (start 96.52 74.7075) (end 96.5675 74.66) (width 0.6) (layer B.Cu) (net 7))
 (segment (start 96.5675 74.66) (end 97.425 74.66) (width 0.6) (layer B.Cu) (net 7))
 (segment (start 94.98 74.66) (end 96.5675 74.66) (width 0.6) (layer B.Cu) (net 7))
 (segment (start 94.9325 74.6125) (end 94.98 74.66) (width 0.6) (layer B.Cu) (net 7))
 (segment (start 93.71 74.6125) (end 94.9325 74.6125) (width 0.6) (layer B.Cu) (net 7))
 (segment (start 92.98 72.7075) (end 92.98 71.8025) (width 0.6) (layer B.Cu) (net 9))
 (segment (start 94.615 70.1675) (end 94.615 69.5325) (width 0.6) (layer B.Cu) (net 9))
 (segment (start 92.98 71.8025) (end 94.615 70.1675) (width 0.6) (layer B.Cu) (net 9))
 (segment (start 91.71 79.01) (end 91.7575 79.0575) (width 0.6) (layer B.Cu) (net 10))
 (segment (start 91.71 76.5175) (end 91.71 79.01) (width 0.6) (layer B.Cu) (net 10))
 (segment (start 96.52 85.09) (end 96.52 87.63) (width 0.6) (layer B.Cu) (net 11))
 (segment (start 102.2825 69.5325) (end 102.2825 68.5325) (width 0.6) (layer B.Cu) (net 13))
 (segment (start 102.87 67.945) (end 102.87 66.675) (width 0.6) (layer B.Cu) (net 13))
 (segment (start 102.2825 68.5325) (end 102.87 67.945) (width 0.6) (layer B.Cu) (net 13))
 (segment (start 100.33 78.74) (end 102.2825 80.6925) (width 0.6) (layer B.Cu) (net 14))
 (segment (start 102.2825 80.6925) (end 102.2825 81.5975) (width 0.6) (layer B.Cu) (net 14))
 (segment (start 100.33 77.47) (end 100.33 78.74) (width 0.6) (layer B.Cu) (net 14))
 (segment (start 97.79 93.345) (end 100.33 93.345) (width 0.6) (layer B.Cu) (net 15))
 (segment (start 103.505 58.1025) (end 103.505 56.515) (width 0.6) (layer B.Cu) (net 16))
 (segment (start 105.41 60.0075) (end 103.505 58.1025) (width 0.6) (layer B.Cu) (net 16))
 (segment (start 105.41 63.135) (end 105.41 60.0075) (width 0.6) (layer B.Cu) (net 16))
 (segment (start 109.22 76.2) (end 109.22 78.74) (width 0.6) (layer B.Cu) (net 18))
 (segment (start 106.68 85.1375) (end 106.68 87.63) (width 0.6) (layer B.Cu) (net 19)))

